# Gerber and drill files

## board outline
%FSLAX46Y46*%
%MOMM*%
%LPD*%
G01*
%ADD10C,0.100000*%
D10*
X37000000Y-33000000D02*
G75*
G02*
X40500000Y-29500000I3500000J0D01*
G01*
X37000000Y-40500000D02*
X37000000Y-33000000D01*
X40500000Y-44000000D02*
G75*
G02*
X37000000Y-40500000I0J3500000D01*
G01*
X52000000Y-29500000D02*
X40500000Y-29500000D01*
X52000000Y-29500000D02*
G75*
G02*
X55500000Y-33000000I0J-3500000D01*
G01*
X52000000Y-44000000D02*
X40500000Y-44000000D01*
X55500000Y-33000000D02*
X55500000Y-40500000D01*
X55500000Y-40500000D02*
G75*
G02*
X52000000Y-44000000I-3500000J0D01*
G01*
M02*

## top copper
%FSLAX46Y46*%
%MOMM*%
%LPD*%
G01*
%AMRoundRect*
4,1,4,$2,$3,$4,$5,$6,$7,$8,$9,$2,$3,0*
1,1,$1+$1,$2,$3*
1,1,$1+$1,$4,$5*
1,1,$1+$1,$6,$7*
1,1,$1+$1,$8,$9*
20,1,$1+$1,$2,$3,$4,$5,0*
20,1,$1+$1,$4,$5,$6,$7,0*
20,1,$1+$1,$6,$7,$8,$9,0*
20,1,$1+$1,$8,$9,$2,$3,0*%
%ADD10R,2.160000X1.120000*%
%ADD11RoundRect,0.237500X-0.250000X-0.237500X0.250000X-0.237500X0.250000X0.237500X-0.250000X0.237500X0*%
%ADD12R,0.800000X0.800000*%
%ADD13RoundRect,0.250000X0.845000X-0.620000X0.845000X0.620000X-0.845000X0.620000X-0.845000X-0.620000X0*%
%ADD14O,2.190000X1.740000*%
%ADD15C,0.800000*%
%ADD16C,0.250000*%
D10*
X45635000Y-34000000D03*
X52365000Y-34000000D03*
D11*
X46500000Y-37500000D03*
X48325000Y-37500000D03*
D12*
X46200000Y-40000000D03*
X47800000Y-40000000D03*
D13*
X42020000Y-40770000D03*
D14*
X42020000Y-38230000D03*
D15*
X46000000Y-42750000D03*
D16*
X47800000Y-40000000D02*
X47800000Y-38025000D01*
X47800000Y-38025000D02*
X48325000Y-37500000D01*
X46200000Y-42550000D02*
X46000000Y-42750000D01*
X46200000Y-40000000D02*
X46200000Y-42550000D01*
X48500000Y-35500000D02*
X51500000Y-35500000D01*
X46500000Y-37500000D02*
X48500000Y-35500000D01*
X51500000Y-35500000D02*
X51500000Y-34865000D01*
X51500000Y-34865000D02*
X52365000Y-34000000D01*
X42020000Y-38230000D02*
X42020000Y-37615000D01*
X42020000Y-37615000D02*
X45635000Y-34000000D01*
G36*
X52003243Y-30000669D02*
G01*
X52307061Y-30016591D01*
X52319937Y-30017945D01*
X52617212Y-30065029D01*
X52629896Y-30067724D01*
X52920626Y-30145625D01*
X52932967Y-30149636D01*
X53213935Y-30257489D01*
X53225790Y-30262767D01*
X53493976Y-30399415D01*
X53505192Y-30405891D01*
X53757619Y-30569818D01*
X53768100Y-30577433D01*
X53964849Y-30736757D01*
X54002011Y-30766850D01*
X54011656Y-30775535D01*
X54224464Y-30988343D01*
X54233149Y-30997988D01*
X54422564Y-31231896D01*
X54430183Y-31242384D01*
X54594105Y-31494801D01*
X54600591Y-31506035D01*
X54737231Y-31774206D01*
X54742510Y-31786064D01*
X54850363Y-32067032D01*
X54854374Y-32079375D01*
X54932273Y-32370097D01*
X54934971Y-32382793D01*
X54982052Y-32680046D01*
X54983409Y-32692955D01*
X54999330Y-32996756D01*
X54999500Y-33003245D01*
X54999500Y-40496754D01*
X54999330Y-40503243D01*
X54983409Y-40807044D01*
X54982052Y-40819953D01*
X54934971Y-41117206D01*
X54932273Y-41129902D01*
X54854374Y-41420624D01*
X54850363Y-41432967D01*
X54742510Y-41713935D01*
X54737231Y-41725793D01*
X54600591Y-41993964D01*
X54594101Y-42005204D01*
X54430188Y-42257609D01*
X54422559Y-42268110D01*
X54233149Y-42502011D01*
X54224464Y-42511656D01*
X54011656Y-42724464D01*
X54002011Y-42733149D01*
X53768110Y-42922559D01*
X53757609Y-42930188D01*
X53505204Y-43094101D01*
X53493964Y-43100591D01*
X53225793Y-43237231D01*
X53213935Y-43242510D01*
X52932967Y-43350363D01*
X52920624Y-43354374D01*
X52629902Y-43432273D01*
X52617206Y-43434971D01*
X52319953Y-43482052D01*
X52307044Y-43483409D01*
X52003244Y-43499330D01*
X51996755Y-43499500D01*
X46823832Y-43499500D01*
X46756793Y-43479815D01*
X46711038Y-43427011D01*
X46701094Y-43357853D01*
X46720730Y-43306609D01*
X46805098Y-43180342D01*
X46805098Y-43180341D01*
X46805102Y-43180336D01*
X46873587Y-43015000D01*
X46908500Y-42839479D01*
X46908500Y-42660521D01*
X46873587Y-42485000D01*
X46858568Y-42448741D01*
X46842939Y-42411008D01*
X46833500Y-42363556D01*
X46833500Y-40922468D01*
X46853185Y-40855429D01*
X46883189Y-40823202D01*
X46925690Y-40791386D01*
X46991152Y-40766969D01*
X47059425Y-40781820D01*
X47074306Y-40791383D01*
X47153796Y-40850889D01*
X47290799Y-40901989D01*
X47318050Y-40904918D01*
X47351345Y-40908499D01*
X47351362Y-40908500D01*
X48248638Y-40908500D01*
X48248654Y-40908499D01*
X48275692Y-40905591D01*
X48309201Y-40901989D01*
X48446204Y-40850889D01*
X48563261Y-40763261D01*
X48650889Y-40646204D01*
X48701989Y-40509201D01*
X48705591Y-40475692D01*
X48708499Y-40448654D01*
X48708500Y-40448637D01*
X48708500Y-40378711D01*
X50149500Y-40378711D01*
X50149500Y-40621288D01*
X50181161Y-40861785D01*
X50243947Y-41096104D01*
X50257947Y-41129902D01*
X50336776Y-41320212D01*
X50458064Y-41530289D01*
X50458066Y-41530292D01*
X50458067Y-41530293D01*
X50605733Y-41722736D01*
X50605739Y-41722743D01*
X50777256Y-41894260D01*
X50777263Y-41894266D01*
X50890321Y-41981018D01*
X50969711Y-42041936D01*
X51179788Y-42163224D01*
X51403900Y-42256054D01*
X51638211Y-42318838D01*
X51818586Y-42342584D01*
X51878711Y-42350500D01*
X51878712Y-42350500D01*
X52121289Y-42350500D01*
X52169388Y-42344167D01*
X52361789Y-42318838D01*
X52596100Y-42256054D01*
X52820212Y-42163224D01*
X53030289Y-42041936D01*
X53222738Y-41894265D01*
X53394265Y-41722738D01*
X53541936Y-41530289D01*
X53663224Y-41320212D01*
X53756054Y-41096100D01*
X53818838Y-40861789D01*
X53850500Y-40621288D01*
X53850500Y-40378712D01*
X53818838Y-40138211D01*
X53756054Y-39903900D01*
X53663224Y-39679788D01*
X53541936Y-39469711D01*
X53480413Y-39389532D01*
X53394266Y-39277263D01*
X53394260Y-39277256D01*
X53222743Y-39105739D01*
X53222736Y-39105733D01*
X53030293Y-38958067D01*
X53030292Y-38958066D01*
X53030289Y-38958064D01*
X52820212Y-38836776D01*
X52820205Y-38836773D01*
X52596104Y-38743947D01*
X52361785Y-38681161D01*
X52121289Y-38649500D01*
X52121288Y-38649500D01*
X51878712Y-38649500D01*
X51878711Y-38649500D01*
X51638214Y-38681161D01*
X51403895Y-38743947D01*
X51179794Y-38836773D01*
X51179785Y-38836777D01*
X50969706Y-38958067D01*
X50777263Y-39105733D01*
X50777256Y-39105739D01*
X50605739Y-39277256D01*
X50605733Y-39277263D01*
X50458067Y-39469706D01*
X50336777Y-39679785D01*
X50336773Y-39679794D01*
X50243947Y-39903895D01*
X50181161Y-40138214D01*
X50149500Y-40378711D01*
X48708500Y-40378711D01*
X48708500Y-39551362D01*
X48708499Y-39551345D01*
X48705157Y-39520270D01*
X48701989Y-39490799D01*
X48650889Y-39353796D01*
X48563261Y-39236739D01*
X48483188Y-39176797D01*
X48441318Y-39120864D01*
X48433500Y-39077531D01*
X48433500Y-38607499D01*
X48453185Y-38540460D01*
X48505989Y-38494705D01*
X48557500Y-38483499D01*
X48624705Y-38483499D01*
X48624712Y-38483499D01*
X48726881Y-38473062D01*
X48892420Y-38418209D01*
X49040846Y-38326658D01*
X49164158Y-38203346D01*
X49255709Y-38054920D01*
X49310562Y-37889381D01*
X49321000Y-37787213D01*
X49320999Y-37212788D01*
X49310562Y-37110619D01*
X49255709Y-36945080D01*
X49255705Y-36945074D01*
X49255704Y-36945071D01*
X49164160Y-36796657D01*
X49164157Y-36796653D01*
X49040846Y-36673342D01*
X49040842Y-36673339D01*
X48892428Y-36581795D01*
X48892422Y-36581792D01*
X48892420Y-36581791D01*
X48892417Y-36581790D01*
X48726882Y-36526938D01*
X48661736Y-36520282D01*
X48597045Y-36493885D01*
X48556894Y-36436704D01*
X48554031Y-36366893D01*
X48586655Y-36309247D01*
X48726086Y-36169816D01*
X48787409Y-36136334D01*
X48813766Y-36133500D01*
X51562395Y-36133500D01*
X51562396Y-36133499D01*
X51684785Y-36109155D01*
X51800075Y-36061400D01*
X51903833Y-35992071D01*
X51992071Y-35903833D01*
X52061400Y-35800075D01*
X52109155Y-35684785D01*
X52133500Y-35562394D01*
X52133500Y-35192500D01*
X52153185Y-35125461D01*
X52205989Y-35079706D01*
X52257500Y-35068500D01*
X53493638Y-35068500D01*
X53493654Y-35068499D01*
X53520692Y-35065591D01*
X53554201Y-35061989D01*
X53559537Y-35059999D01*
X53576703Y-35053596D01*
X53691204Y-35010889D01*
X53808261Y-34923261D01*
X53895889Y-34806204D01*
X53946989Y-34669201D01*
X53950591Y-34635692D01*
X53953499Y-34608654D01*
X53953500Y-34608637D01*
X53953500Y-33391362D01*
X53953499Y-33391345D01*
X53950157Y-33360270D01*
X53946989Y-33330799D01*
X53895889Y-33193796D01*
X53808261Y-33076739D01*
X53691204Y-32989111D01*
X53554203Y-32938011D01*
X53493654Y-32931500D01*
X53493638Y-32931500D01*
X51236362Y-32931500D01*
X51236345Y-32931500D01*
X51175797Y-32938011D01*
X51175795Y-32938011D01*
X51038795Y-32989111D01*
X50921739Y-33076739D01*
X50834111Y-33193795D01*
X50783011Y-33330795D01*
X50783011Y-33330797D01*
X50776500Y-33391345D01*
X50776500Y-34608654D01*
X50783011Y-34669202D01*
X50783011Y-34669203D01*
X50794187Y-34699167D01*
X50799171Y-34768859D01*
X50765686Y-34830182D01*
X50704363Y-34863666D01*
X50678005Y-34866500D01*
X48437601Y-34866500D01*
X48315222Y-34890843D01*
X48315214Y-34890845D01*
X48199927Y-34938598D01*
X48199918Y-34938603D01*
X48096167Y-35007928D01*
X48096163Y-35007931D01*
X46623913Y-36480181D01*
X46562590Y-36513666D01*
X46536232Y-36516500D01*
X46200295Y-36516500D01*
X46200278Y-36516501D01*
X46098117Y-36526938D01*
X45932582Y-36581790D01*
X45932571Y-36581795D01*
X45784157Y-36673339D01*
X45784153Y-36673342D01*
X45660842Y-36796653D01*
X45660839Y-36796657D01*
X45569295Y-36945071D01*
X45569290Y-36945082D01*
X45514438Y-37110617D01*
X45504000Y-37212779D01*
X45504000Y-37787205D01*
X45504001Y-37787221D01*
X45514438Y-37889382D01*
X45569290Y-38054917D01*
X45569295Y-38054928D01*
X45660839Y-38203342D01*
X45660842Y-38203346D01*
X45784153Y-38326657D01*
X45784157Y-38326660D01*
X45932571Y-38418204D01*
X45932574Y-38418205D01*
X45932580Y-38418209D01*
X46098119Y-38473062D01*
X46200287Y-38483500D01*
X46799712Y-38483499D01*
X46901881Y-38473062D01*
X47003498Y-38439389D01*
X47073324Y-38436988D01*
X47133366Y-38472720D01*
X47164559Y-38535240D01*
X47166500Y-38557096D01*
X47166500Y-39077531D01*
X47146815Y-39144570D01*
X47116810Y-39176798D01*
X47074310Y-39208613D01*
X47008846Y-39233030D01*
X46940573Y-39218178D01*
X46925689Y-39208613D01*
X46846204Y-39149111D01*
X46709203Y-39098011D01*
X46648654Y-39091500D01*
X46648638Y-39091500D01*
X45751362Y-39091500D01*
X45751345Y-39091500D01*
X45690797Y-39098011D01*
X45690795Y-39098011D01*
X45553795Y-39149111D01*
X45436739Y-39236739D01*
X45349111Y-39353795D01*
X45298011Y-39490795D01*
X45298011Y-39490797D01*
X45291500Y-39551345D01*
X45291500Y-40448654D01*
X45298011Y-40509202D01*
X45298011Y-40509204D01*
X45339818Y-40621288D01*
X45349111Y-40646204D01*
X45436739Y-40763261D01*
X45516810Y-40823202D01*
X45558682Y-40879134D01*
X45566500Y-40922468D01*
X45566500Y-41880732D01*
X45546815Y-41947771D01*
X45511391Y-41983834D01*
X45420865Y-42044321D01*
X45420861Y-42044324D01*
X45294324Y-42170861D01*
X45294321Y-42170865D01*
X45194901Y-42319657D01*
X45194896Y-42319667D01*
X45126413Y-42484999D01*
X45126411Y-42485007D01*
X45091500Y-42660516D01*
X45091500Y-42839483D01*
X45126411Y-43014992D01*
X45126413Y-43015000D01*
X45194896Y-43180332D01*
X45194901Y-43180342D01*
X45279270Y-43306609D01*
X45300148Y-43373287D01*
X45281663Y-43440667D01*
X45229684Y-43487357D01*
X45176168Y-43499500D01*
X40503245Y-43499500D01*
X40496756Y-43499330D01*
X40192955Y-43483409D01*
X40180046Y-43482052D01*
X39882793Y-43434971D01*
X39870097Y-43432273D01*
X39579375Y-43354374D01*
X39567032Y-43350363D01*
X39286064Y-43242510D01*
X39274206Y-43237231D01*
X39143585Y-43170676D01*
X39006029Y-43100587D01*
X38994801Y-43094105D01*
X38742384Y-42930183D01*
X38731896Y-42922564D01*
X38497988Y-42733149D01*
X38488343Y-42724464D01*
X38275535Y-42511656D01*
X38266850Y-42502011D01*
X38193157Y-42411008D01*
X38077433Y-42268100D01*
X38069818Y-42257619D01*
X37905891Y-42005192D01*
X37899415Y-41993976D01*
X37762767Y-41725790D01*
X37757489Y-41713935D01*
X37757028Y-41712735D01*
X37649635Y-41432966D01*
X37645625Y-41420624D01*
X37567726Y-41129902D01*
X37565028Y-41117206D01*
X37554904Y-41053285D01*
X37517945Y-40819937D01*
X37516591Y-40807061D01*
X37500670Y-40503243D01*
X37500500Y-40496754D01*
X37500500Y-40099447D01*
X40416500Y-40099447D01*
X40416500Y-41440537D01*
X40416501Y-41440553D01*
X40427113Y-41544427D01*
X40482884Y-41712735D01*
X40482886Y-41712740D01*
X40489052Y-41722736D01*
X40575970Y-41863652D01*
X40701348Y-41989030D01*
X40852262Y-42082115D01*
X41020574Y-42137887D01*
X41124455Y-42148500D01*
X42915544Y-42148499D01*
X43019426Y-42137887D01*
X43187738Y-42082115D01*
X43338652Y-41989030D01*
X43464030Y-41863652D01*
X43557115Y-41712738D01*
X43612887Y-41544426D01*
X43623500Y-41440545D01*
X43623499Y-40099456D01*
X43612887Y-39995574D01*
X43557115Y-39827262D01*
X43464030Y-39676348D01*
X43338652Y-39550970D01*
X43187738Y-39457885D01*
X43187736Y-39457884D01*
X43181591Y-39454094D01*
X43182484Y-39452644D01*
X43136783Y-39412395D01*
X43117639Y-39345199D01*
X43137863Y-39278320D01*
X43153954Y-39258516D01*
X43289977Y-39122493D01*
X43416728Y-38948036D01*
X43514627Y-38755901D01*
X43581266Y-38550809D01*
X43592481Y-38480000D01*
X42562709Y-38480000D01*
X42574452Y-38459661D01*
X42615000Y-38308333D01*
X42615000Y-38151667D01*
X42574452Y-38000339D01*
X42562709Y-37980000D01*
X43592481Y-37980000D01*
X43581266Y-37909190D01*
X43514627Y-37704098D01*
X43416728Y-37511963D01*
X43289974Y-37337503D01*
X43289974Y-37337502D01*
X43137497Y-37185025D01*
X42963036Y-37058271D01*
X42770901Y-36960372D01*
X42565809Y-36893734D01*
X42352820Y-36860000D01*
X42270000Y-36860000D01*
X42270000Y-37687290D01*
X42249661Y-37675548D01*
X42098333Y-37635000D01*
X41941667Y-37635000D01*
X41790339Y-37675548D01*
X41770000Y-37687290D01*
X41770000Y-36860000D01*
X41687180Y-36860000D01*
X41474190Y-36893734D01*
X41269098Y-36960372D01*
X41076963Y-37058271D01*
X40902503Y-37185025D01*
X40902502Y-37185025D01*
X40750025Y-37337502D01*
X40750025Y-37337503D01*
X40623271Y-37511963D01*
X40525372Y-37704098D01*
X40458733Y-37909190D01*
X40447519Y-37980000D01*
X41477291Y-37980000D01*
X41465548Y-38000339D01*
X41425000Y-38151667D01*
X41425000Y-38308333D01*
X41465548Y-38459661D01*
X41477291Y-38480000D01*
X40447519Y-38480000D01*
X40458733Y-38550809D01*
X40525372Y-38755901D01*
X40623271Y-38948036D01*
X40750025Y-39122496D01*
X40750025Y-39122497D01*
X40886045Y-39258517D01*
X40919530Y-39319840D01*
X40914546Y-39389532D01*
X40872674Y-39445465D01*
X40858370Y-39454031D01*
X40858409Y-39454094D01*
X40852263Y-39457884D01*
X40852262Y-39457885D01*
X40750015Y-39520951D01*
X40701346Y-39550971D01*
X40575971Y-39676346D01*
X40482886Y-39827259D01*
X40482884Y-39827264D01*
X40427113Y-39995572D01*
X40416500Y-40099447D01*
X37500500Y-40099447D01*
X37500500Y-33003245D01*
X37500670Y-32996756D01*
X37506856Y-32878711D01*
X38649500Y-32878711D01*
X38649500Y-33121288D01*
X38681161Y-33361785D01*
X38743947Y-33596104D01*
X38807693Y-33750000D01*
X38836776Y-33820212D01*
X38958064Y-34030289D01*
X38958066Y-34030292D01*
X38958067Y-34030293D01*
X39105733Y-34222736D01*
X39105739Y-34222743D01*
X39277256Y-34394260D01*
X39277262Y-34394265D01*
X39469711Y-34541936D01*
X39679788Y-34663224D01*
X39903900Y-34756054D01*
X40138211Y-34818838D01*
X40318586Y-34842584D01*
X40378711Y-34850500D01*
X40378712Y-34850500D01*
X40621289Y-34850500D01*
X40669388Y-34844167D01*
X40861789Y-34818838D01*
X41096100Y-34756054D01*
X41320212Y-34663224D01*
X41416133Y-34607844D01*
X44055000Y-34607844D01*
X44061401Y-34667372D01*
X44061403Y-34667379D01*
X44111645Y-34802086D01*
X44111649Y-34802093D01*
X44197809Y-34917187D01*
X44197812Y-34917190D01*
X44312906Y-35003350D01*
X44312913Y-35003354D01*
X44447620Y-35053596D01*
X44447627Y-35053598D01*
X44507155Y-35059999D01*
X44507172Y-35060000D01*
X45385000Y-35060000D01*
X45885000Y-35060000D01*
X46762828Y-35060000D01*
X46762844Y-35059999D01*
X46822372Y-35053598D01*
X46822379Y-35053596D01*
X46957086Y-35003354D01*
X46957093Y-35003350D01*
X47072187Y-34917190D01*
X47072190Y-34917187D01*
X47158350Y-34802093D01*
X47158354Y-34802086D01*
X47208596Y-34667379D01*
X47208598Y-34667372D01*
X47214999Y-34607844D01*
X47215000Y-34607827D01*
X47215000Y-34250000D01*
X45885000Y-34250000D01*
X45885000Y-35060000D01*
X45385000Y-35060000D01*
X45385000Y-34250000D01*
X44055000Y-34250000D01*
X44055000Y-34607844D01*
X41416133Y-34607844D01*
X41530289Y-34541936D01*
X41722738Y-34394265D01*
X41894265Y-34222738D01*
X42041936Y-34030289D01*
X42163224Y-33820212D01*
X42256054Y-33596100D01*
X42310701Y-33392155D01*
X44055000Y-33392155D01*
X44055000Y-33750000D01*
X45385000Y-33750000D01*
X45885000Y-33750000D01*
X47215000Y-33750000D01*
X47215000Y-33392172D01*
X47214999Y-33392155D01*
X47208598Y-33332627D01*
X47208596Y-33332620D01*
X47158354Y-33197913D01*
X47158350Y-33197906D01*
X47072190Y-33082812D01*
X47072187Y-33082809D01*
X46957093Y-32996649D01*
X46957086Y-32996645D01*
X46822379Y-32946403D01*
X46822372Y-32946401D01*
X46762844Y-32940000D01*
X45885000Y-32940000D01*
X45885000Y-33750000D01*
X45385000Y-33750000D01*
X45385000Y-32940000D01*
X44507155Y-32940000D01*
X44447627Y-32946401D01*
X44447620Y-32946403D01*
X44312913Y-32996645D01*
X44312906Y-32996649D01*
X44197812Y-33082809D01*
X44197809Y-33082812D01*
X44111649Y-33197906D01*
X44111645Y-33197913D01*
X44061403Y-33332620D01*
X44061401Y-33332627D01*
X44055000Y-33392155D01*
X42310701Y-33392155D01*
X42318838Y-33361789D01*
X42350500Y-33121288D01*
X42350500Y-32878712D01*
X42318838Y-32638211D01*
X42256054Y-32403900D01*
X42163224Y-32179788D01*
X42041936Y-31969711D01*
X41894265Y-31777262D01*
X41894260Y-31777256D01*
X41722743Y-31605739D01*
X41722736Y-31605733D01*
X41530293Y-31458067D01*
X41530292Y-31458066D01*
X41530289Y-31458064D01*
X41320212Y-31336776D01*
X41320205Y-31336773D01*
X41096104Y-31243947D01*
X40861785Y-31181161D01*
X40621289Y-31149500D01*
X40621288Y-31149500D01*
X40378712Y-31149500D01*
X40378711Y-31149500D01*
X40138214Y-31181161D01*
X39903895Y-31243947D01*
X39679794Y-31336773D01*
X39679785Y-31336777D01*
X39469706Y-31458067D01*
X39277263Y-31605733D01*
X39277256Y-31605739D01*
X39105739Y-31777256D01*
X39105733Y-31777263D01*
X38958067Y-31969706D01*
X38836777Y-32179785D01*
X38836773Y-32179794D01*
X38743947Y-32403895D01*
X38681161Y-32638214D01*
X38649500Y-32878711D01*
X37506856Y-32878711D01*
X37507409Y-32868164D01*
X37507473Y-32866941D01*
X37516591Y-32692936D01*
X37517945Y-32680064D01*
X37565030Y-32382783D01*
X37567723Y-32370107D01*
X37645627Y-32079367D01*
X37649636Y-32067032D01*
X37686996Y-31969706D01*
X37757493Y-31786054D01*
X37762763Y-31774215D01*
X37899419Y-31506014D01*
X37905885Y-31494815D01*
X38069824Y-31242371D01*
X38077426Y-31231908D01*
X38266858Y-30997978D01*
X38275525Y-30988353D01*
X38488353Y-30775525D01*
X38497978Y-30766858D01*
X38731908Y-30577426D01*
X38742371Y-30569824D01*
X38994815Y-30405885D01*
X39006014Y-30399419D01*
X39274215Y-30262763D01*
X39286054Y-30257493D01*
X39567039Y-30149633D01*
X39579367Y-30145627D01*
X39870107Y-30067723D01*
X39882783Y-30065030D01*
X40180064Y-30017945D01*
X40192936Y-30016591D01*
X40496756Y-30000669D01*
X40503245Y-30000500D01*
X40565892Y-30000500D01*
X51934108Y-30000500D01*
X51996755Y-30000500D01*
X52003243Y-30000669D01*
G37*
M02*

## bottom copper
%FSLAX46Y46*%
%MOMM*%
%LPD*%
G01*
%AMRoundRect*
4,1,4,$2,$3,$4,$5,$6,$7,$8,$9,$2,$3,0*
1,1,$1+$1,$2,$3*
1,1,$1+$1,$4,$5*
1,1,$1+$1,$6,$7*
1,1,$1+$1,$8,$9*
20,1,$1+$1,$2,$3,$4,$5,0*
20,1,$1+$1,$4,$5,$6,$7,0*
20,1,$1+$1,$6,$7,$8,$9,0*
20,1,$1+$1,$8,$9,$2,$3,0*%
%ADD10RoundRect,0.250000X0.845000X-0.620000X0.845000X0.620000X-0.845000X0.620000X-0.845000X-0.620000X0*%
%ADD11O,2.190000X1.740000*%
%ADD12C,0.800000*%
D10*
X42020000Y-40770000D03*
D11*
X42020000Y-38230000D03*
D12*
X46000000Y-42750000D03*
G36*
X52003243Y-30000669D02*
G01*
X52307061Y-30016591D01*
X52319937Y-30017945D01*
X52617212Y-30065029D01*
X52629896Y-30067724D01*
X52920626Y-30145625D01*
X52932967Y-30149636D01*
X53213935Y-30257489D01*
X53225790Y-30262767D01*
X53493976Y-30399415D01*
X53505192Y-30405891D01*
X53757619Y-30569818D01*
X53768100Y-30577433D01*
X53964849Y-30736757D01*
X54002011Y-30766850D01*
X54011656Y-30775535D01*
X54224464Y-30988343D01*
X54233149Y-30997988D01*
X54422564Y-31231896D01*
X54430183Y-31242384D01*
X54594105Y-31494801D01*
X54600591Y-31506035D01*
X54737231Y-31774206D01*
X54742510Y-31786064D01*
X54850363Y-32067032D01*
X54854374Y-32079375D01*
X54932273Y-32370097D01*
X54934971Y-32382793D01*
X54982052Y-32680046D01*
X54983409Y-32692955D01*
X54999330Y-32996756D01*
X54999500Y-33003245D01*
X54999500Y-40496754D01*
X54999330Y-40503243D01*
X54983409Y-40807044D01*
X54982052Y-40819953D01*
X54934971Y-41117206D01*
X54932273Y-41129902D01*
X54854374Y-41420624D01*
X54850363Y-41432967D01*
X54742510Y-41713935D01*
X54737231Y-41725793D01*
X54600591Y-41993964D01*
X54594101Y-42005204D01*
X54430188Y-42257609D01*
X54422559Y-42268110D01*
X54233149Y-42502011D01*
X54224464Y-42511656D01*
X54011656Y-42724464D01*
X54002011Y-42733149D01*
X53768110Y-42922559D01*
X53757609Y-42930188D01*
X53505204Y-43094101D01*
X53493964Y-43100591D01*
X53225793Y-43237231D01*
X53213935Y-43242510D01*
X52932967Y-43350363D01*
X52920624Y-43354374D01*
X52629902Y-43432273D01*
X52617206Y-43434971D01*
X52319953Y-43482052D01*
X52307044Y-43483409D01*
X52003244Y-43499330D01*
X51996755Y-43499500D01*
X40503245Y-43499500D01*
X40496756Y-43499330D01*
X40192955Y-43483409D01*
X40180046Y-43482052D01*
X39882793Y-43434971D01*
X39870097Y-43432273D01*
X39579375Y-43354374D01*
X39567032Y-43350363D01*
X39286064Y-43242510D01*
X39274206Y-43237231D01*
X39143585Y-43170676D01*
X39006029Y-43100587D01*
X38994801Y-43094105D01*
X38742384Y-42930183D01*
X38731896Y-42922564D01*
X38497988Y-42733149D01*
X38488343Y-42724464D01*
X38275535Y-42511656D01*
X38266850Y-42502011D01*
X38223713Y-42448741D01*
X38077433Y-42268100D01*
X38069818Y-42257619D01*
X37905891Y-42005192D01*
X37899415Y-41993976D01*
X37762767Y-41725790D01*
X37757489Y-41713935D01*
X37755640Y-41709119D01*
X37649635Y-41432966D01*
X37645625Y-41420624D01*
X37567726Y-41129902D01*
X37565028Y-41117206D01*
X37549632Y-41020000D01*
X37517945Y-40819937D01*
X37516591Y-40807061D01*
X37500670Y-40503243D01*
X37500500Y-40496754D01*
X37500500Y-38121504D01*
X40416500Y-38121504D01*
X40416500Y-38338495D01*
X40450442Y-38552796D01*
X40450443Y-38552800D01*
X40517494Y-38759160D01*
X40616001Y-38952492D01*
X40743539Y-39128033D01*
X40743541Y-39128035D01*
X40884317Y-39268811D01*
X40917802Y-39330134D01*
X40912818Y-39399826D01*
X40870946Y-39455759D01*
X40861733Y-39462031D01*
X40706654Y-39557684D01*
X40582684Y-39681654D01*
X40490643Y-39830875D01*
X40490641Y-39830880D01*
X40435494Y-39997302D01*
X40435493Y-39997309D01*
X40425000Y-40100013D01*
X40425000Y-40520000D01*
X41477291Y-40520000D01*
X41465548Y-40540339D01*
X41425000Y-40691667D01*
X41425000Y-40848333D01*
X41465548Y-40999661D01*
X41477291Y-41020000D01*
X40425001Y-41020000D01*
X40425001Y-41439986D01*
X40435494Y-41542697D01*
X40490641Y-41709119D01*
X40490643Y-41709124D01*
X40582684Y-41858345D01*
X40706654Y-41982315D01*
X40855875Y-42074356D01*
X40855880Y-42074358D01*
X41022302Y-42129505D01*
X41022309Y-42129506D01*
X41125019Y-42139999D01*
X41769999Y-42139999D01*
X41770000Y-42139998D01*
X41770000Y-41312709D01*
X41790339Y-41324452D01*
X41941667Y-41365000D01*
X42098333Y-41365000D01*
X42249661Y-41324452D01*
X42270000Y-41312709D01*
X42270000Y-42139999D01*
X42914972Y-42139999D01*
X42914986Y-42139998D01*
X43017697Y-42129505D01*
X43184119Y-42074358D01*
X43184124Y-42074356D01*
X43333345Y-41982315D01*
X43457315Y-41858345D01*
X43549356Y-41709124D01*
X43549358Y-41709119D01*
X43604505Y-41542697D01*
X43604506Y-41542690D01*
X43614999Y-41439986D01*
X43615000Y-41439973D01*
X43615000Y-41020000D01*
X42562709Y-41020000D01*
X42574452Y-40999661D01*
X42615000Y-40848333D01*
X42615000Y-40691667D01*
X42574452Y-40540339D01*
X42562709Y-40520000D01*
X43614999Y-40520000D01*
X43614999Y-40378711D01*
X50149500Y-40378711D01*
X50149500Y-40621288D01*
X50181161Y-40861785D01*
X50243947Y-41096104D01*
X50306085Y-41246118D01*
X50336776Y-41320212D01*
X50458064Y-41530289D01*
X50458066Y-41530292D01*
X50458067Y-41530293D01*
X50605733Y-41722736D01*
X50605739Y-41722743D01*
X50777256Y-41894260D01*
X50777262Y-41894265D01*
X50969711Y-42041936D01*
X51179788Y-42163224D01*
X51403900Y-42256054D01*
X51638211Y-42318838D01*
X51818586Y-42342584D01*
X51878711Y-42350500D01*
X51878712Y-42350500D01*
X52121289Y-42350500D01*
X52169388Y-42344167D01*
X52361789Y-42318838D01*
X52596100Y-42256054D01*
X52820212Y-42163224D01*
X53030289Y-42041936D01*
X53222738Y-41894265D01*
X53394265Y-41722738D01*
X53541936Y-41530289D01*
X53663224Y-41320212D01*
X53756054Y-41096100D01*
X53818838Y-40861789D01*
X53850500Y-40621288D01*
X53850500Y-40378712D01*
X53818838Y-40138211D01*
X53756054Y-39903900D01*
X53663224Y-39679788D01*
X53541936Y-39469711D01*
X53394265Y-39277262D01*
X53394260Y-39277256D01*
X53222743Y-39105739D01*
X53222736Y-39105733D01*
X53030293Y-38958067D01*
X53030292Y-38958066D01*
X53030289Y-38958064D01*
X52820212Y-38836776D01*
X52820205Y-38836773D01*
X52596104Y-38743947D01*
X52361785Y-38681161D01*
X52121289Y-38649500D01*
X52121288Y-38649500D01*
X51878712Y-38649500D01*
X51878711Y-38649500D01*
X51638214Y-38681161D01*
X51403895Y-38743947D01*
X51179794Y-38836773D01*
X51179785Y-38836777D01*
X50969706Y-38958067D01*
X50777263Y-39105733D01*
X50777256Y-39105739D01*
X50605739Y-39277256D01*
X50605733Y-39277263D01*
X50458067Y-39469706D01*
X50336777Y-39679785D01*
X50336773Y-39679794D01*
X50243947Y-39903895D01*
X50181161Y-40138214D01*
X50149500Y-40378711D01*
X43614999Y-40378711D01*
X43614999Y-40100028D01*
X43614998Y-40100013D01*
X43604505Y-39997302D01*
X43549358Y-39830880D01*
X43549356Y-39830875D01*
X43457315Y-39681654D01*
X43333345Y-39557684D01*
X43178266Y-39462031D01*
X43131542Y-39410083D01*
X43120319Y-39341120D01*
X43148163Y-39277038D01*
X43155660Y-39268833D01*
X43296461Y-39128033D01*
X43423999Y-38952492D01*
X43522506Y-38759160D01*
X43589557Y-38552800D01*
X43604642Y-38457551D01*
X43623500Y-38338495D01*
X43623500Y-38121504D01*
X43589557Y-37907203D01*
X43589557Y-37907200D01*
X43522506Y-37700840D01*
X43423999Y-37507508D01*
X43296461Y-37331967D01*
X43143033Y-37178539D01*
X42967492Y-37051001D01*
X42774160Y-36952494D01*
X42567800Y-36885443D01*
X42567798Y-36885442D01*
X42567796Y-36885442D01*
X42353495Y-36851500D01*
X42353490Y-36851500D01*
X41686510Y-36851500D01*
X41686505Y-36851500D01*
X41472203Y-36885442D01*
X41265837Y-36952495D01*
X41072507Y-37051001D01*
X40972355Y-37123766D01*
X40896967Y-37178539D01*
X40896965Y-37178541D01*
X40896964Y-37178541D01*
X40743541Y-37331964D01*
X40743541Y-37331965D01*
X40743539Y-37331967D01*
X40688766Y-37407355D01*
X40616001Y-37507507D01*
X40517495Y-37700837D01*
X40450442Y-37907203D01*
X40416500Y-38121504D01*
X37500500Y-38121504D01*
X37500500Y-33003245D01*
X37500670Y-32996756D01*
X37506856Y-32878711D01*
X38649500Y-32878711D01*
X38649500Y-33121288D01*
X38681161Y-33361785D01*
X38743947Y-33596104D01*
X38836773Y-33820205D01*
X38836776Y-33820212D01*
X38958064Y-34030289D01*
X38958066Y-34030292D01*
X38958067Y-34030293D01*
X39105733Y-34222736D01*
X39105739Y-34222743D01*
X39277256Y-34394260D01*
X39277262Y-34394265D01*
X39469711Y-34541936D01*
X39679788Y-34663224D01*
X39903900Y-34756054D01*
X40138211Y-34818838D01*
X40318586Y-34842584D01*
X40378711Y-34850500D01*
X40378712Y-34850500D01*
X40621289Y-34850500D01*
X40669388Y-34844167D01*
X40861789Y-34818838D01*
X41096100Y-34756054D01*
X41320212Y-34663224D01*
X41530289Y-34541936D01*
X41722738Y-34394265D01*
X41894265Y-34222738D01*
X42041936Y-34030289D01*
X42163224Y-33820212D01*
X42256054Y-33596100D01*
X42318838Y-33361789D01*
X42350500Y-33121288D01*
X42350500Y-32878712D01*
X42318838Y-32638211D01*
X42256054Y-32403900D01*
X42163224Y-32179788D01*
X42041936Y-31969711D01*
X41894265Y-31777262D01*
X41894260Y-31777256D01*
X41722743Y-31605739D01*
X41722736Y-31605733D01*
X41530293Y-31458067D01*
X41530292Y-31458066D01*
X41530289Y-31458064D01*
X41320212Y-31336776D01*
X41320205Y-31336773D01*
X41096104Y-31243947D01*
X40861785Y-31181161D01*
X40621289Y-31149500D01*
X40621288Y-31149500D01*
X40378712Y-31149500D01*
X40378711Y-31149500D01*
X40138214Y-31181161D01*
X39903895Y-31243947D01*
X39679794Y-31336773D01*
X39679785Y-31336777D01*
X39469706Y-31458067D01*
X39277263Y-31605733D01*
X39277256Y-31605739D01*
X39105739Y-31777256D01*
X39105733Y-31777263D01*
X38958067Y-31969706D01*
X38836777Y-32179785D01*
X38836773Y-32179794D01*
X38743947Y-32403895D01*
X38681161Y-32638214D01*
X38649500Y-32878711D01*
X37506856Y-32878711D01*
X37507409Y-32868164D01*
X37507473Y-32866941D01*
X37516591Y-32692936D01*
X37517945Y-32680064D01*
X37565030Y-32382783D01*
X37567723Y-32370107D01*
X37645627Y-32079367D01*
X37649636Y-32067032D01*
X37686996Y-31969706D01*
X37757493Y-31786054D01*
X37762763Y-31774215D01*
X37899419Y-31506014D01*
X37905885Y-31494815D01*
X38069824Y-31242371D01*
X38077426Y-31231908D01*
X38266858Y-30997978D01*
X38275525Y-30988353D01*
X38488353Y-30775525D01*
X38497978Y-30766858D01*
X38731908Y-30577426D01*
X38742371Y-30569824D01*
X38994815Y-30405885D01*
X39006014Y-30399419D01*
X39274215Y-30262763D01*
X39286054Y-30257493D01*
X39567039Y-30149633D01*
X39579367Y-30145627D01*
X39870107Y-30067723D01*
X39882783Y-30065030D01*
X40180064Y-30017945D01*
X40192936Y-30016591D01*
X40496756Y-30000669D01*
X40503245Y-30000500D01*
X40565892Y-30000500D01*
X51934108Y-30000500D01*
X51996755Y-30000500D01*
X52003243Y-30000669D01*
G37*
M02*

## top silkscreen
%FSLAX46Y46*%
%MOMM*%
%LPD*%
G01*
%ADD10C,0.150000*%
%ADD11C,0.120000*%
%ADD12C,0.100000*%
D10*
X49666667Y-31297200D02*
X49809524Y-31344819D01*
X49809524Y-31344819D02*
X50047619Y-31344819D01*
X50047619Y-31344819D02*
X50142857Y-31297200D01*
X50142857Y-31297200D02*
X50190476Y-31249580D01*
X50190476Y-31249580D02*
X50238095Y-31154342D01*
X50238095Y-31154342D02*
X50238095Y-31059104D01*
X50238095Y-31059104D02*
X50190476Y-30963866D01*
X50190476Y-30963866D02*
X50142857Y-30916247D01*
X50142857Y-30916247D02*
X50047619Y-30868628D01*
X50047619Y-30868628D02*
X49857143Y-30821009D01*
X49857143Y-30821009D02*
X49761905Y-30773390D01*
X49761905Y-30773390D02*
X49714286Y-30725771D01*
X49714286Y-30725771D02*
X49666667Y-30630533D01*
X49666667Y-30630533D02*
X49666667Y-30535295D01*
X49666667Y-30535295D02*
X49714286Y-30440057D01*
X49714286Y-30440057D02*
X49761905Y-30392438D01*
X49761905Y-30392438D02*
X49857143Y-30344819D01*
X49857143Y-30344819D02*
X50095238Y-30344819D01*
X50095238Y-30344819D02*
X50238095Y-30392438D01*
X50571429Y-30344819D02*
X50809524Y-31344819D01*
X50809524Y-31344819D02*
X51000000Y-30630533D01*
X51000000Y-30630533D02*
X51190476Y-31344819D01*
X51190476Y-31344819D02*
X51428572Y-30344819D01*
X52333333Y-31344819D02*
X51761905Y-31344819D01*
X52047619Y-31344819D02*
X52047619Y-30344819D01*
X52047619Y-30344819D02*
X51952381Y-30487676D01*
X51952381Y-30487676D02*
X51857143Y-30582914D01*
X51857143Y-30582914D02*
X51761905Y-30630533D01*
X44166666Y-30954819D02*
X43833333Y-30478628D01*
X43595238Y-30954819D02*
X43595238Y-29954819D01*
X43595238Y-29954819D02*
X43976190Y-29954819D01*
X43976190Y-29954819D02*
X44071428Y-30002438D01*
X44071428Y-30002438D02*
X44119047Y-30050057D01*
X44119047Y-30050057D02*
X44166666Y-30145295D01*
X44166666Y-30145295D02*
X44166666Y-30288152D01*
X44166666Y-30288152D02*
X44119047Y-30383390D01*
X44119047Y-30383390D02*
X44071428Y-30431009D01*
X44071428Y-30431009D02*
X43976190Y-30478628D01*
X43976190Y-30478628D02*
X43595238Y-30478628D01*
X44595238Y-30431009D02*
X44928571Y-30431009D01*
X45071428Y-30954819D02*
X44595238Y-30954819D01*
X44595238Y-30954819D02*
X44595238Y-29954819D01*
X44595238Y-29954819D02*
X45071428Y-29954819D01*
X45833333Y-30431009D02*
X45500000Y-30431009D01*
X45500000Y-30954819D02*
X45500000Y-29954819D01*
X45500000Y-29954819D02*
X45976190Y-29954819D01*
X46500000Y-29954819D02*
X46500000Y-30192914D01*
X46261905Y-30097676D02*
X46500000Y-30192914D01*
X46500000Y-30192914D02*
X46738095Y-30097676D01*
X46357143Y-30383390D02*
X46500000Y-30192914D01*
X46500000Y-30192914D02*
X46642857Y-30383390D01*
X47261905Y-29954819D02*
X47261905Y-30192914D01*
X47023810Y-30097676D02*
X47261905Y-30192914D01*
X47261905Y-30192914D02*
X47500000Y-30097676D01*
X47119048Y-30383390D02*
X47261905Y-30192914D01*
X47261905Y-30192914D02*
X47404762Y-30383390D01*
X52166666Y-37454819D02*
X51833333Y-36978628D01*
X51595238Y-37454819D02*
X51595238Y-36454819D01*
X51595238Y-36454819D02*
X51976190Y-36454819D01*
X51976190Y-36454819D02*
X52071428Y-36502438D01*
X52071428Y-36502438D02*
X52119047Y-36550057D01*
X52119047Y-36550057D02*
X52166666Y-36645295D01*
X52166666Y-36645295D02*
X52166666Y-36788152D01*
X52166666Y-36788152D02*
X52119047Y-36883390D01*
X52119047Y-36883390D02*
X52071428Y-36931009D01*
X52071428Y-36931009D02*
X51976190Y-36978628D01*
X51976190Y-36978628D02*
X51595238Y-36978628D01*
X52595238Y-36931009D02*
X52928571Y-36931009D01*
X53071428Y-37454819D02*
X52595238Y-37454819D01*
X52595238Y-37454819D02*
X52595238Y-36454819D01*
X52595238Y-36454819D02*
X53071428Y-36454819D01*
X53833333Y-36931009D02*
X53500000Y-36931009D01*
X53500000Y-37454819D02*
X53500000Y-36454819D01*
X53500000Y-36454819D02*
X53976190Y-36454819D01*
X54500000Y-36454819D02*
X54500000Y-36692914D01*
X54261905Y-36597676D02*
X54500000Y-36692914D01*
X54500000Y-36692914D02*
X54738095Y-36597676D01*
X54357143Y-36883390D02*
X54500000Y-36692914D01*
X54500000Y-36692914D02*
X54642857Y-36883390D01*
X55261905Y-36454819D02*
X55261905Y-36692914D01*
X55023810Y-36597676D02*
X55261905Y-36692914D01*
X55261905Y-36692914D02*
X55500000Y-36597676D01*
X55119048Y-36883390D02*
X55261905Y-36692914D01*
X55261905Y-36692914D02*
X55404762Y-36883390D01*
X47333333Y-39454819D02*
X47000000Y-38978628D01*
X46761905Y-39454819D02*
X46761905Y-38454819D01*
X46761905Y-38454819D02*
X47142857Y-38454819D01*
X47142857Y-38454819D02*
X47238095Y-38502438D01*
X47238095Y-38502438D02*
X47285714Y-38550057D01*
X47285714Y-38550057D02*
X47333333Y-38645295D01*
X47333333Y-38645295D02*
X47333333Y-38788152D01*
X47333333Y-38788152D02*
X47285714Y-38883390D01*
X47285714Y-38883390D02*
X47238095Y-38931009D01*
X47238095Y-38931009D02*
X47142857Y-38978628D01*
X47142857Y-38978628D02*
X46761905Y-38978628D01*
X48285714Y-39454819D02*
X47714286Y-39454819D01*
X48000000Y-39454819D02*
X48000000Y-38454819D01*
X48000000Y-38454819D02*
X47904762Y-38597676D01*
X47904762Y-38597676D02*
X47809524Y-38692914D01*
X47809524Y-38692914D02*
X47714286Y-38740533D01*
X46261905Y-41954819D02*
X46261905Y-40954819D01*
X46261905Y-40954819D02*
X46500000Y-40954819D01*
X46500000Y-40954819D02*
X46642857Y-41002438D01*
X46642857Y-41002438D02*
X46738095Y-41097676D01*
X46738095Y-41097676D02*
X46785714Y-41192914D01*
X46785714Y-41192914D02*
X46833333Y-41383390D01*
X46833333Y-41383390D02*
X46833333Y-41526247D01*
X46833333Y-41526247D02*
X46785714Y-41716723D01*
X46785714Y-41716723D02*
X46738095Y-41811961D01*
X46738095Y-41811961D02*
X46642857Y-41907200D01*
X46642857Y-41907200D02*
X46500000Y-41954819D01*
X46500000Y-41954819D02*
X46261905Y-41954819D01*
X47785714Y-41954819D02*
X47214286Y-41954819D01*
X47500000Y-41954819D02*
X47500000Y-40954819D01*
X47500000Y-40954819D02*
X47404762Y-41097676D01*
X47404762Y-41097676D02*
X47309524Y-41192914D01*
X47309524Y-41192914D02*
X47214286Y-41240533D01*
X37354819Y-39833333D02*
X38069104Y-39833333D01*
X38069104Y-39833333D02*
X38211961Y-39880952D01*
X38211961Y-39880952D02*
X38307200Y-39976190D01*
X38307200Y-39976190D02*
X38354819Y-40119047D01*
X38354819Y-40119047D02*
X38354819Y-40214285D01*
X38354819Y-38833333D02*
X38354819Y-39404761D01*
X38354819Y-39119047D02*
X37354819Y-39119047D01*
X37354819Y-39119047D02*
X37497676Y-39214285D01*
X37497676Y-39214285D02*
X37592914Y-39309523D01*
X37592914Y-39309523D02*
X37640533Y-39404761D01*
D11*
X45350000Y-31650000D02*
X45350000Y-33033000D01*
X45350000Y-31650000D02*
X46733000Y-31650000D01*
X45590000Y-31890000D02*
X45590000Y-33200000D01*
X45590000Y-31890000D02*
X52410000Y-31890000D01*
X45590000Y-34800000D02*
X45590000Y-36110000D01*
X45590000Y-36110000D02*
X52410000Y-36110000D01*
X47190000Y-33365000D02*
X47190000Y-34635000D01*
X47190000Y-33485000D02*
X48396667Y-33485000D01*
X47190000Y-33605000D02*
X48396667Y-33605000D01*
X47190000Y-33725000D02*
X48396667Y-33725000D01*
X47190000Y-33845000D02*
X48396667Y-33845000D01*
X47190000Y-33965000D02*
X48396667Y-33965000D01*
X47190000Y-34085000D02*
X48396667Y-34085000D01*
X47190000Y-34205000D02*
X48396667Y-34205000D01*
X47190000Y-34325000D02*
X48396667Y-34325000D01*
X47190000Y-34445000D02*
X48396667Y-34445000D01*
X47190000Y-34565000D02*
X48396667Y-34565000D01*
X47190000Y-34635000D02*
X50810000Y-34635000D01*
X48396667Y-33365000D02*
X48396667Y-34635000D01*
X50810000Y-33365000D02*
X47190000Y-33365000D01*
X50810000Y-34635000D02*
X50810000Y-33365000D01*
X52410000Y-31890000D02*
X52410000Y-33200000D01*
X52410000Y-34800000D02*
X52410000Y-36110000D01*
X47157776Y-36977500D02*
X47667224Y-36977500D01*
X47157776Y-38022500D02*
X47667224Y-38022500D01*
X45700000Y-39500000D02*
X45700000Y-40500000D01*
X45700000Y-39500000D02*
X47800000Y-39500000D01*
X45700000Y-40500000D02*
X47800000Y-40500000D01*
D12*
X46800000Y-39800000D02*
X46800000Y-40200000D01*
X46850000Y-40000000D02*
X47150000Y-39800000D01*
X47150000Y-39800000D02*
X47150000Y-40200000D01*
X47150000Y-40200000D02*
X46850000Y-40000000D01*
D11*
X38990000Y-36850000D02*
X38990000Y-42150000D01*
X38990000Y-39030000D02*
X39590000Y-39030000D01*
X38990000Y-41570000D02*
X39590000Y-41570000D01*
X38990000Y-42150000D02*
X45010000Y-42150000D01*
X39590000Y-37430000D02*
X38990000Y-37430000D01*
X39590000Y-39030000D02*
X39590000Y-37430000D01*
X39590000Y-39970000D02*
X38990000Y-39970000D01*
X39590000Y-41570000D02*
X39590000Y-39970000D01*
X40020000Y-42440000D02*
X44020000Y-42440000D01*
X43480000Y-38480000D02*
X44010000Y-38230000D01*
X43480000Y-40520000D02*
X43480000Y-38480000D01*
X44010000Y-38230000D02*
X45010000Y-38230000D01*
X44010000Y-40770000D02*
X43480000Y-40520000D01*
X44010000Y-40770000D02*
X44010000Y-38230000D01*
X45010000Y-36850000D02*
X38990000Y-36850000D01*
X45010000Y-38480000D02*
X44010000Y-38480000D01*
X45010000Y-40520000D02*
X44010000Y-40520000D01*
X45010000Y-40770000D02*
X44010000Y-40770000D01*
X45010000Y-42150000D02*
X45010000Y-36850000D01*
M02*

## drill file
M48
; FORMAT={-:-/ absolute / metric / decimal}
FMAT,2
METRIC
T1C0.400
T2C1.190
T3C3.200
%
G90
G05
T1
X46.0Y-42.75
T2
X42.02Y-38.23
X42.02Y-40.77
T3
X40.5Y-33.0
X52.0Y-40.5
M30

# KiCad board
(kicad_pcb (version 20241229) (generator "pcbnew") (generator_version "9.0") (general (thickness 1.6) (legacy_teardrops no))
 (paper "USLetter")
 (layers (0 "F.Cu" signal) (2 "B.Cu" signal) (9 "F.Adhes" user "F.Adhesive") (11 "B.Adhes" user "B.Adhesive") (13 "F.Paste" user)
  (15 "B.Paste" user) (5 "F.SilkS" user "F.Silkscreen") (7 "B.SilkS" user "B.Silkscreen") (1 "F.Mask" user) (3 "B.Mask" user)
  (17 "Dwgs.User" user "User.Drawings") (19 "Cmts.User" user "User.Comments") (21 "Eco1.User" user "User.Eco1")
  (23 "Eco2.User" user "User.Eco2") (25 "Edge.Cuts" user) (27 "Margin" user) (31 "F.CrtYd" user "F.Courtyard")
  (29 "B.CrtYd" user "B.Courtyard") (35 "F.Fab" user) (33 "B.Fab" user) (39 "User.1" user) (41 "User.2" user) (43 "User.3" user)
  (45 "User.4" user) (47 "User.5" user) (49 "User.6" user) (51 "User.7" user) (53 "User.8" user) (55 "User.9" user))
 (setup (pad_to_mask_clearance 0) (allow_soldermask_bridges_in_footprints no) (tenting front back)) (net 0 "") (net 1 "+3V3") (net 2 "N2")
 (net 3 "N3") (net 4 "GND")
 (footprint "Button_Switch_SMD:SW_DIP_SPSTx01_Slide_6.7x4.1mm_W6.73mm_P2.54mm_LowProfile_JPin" (layer "F.Cu") (at 49 34)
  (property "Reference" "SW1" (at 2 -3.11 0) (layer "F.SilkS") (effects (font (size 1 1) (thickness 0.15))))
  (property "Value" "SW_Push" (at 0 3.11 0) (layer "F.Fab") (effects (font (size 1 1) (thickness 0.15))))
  (fp_line (start -3.65 -2.35) (end -3.65 -0.967) (stroke (width 0.12) (type solid)) (layer "F.SilkS"))
  (fp_line (start -3.65 -2.35) (end -2.267 -2.35) (stroke (width 0.12) (type solid)) (layer "F.SilkS"))
  (fp_line (start -3.41 -2.11) (end -3.41 -0.8) (stroke (width 0.12) (type solid)) (layer "F.SilkS"))
  (fp_line (start -3.41 -2.11) (end 3.41 -2.11) (stroke (width 0.12) (type solid)) (layer "F.SilkS"))
  (fp_line (start -3.41 0.8) (end -3.41 2.11) (stroke (width 0.12) (type solid)) (layer "F.SilkS"))
  (fp_line (start -3.41 2.11) (end 3.41 2.11) (stroke (width 0.12) (type solid)) (layer "F.SilkS"))
  (fp_line (start -1.81 -0.635) (end -1.81 0.635) (stroke (width 0.12) (type solid)) (layer "F.SilkS"))
  (fp_line (start -1.81 -0.515) (end -0.603333 -0.515) (stroke (width 0.12) (type solid)) (layer "F.SilkS"))
  (fp_line (start -1.81 -0.395) (end -0.603333 -0.395) (stroke (width 0.12) (type solid)) (layer "F.SilkS"))
  (fp_line (start -1.81 -0.275) (end -0.603333 -0.275) (stroke (width 0.12) (type solid)) (layer "F.SilkS"))
  (fp_line (start -1.81 -0.155) (end -0.603333 -0.155) (stroke (width 0.12) (type solid)) (layer "F.SilkS"))
  (fp_line (start -1.81 -0.035) (end -0.603333 -0.035) (stroke (width 0.12) (type solid)) (layer "F.SilkS"))
  (fp_line (start -1.81 0.085) (end -0.603333 0.085) (stroke (width 0.12) (type solid)) (layer "F.SilkS"))
  (fp_line (start -1.81 0.205) (end -0.603333 0.205) (stroke (width 0.12) (type solid)) (layer "F.SilkS"))
  (fp_line (start -1.81 0.325) (end -0.603333 0.325) (stroke (width 0.12) (type solid)) (layer "F.SilkS"))
  (fp_line (start -1.81 0.445) (end -0.603333 0.445) (stroke (width 0.12) (type solid)) (layer "F.SilkS"))
  (fp_line (start -1.81 0.565) (end -0.603333 0.565) (stroke (width 0.12) (type solid)) (layer "F.SilkS"))
  (fp_line (start -1.81 0.635) (end 1.81 0.635) (stroke (width 0.12) (type solid)) (layer "F.SilkS"))
  (fp_line (start -0.603333 -0.635) (end -0.603333 0.635) (stroke (width 0.12) (type solid)) (layer "F.SilkS"))
  (fp_line (start 1.81 -0.635) (end -1.81 -0.635) (stroke (width 0.12) (type solid)) (layer "F.SilkS"))
  (fp_line (start 1.81 0.635) (end 1.81 -0.635) (stroke (width 0.12) (type solid)) (layer "F.SilkS"))
  (fp_line (start 3.41 -2.11) (end 3.41 -0.8) (stroke (width 0.12) (type solid)) (layer "F.SilkS"))
  (fp_line (start 3.41 0.8) (end 3.41 2.11) (stroke (width 0.12) (type solid)) (layer "F.SilkS"))
  (pad "1" smd rect (at -3.365 0) (size 2.16 1.12) (layers "F.Cu" "F.Mask" "F.Paste") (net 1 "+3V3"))
  (pad "2" smd rect (at 3.365 0) (size 2.16 1.12) (layers "F.Cu" "F.Mask" "F.Paste") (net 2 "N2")))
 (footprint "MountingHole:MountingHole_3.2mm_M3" (layer "F.Cu") (at 40.5 33)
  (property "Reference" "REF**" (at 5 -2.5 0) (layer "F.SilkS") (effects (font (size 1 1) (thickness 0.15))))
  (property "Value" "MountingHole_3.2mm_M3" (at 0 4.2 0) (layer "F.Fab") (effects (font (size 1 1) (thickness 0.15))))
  (pad "" np_thru_hole circle (at 0 0) (size 3.2 3.2) (drill 3.2) (layers "*.Cu" "*.Mask")))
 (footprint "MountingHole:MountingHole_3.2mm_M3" (layer "F.Cu") (at 52 40.5)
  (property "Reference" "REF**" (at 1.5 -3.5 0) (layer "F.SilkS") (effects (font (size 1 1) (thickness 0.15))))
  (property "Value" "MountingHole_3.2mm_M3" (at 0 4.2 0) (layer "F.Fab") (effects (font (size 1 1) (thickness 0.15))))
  (pad "" np_thru_hole circle (at 0 0) (size 3.2 3.2) (drill 3.2) (layers "*.Cu" "*.Mask")))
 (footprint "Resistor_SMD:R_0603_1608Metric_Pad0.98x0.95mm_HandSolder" (layer "F.Cu") (at 47.4125 37.5)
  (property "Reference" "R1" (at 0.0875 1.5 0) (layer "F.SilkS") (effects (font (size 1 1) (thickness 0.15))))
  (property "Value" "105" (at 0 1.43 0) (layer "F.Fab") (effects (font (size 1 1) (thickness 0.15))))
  (fp_line (start -0.254724 -0.5225) (end 0.254724 -0.5225) (stroke (width 0.12) (type solid)) (layer "F.SilkS"))
  (fp_line (start -0.254724 0.5225) (end 0.254724 0.5225) (stroke (width 0.12) (type solid)) (layer "F.SilkS"))
  (pad "1" smd roundrect (at -0.9125 0) (size 0.975 0.95) (layers "F.Cu" "F.Mask" "F.Paste") (roundrect_rratio 0.25) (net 2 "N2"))
  (pad "2" smd roundrect (at 0.9125 0) (size 0.975 0.95) (layers "F.Cu" "F.Mask" "F.Paste") (roundrect_rratio 0.25) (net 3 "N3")))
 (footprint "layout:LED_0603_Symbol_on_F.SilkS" (layer "F.Cu") (at 47 40)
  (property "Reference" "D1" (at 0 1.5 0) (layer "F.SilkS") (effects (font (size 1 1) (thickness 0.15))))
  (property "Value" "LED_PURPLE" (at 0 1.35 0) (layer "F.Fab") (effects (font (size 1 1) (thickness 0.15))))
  (fp_line (start -1.3 -0.5) (end -1.3 0.5) (stroke (width 0.12) (type solid)) (layer "F.SilkS"))
  (fp_line (start -1.3 -0.5) (end 0.8 -0.5) (stroke (width 0.12) (type solid)) (layer "F.SilkS"))
  (fp_line (start -1.3 0.5) (end 0.8 0.5) (stroke (width 0.12) (type solid)) (layer "F.SilkS"))
  (fp_line (start -0.2 -0.2) (end -0.2 0.2) (stroke (width 0.1) (type solid)) (layer "F.SilkS"))
  (fp_line (start -0.15 0) (end 0.15 -0.2) (stroke (width 0.1) (type solid)) (layer "F.SilkS"))
  (fp_line (start 0.15 -0.2) (end 0.15 0.2) (stroke (width 0.1) (type solid)) (layer "F.SilkS"))
  (fp_line (start 0.15 0.2) (end -0.15 0) (stroke (width 0.1) (type solid)) (layer "F.SilkS"))
  (pad "1" smd rect (at -0.8 0 180) (size 0.8 0.8) (layers "F.Cu" "F.Mask" "F.Paste") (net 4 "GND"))
  (pad "2" smd rect (at 0.8 0 180) (size 0.8 0.8) (layers "F.Cu" "F.Mask" "F.Paste") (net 3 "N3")))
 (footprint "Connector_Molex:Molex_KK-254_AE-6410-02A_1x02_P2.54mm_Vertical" (layer "F.Cu") (at 42.02 40.77 90)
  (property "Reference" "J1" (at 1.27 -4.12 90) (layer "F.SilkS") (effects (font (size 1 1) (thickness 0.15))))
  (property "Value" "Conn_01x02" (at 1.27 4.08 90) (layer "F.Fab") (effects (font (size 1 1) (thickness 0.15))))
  (fp_line (start 3.92 -3.03) (end -1.38 -3.03) (stroke (width 0.12) (type solid)) (layer "F.SilkS"))
  (fp_line (start 1.74 -3.03) (end 1.74 -2.43) (stroke (width 0.12) (type solid)) (layer "F.SilkS"))
  (fp_line (start -0.8 -3.03) (end -0.8 -2.43) (stroke (width 0.12) (type solid)) (layer "F.SilkS"))
  (fp_line (start -1.38 -3.03) (end -1.38 2.99) (stroke (width 0.12) (type solid)) (layer "F.SilkS"))
  (fp_line (start 3.34 -2.43) (end 3.34 -3.03) (stroke (width 0.12) (type solid)) (layer "F.SilkS"))
  (fp_line (start 1.74 -2.43) (end 3.34 -2.43) (stroke (width 0.12) (type solid)) (layer "F.SilkS"))
  (fp_line (start 0.8 -2.43) (end 0.8 -3.03) (stroke (width 0.12) (type solid)) (layer "F.SilkS"))
  (fp_line (start -0.8 -2.43) (end 0.8 -2.43) (stroke (width 0.12) (type solid)) (layer "F.SilkS"))
  (fp_line (start -1.67 -2) (end -1.67 2) (stroke (width 0.12) (type solid)) (layer "F.SilkS"))
  (fp_line (start 2.29 1.46) (end 2.54 1.99) (stroke (width 0.12) (type solid)) (layer "F.SilkS"))
  (fp_line (start 0.25 1.46) (end 2.29 1.46) (stroke (width 0.12) (type solid)) (layer "F.SilkS"))
  (fp_line (start 2.54 1.99) (end 2.54 2.99) (stroke (width 0.12) (type solid)) (layer "F.SilkS"))
  (fp_line (start 0 1.99) (end 0.25 1.46) (stroke (width 0.12) (type solid)) (layer "F.SilkS"))
  (fp_line (start 0 1.99) (end 2.54 1.99) (stroke (width 0.12) (type solid)) (layer "F.SilkS"))
  (fp_line (start 3.92 2.99) (end 3.92 -3.03) (stroke (width 0.12) (type solid)) (layer "F.SilkS"))
  (fp_line (start 2.29 2.99) (end 2.29 1.99) (stroke (width 0.12) (type solid)) (layer "F.SilkS"))
  (fp_line (start 0.25 2.99) (end 0.25 1.99) (stroke (width 0.12) (type solid)) (layer "F.SilkS"))
  (fp_line (start 0 2.99) (end 0 1.99) (stroke (width 0.12) (type solid)) (layer "F.SilkS"))
  (fp_line (start -1.38 2.99) (end 3.92 2.99) (stroke (width 0.12) (type solid)) (layer "F.SilkS"))
  (pad "1" thru_hole roundrect (at 0 0 90) (size 1.74 2.19) (drill 1.19) (layers "*.Cu" "*.Mask") (remove_unused_layers no)
   (roundrect_rratio 0.143678) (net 4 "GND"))
  (pad "2" thru_hole oval (at 2.54 0 90) (size 1.74 2.19) (drill 1.19) (layers "*.Cu" "*.Mask") (remove_unused_layers no) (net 1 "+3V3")))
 (gr_arc (start 37 33) (mid 38.025126 30.525126) (end 40.5 29.5) (stroke (width 0.1) (type default)) (layer "Edge.Cuts"))
 (gr_line (start 37 40.5) (end 37 33) (stroke (width 0.1) (type default)) (layer "Edge.Cuts"))
 (gr_arc (start 40.5 44) (mid 38.025126 42.974874) (end 37 40.5) (stroke (width 0.1) (type default)) (layer "Edge.Cuts"))
 (gr_line (start 52 29.5) (end 40.5 29.5) (stroke (width 0.1) (type default)) (layer "Edge.Cuts"))
 (gr_arc (start 52 29.5) (mid 54.474874 30.525126) (end 55.5 33) (stroke (width 0.1) (type default)) (layer "Edge.Cuts"))
 (gr_line (start 52 44) (end 40.5 44) (stroke (width 0.1) (type default)) (layer "Edge.Cuts"))
 (gr_line (start 55.5 33) (end 55.5 40.5) (stroke (width 0.1) (type default)) (layer "Edge.Cuts"))
 (gr_arc (start 55.5 40.5) (mid 54.474874 42.974874) (end 52 44) (stroke (width 0.1) (type default)) (layer "Edge.Cuts"))
 (segment (start 47.8 40) (end 47.8 38.025) (width 0.25) (layer "F.Cu") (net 3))
 (segment (start 47.8 38.025) (end 48.325 37.5) (width 0.25) (layer "F.Cu") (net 3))
 (segment (start 46.2 42.55) (end 46 42.75) (width 0.25) (layer "F.Cu") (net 4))
 (segment (start 46.2 40) (end 46.2 42.55) (width 0.25) (layer "F.Cu") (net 4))
 (via (at 46 42.75) (size 0.8) (drill 0.4) (layers "F.Cu" "B.Cu") (free yes) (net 4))
 (segment (start 48.5 35.5) (end 51.5 35.5) (width 0.25) (layer "F.Cu") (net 2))
 (segment (start 46.5 37.5) (end 48.5 35.5) (width 0.25) (layer "F.Cu") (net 2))
 (segment (start 51.5 35.5) (end 51.5 34.865) (width 0.25) (layer "F.Cu") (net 2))
 (segment (start 51.5 34.865) (end 52.365 34) (width 0.25) (layer "F.Cu") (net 2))
 (segment (start 42.02 38.23) (end 42.02 37.615) (width 0.25) (layer "F.Cu") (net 1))
 (segment (start 42.02 37.615) (end 45.635 34) (width 0.25) (layer "F.Cu") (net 1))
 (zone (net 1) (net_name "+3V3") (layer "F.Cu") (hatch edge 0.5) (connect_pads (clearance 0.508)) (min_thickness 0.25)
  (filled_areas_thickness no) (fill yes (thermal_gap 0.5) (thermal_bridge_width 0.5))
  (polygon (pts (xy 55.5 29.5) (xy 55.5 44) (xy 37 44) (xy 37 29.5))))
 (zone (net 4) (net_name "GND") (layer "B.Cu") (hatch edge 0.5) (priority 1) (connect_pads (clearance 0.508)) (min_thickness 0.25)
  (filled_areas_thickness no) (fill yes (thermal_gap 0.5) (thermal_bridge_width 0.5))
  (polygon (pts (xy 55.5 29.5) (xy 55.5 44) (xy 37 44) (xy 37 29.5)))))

